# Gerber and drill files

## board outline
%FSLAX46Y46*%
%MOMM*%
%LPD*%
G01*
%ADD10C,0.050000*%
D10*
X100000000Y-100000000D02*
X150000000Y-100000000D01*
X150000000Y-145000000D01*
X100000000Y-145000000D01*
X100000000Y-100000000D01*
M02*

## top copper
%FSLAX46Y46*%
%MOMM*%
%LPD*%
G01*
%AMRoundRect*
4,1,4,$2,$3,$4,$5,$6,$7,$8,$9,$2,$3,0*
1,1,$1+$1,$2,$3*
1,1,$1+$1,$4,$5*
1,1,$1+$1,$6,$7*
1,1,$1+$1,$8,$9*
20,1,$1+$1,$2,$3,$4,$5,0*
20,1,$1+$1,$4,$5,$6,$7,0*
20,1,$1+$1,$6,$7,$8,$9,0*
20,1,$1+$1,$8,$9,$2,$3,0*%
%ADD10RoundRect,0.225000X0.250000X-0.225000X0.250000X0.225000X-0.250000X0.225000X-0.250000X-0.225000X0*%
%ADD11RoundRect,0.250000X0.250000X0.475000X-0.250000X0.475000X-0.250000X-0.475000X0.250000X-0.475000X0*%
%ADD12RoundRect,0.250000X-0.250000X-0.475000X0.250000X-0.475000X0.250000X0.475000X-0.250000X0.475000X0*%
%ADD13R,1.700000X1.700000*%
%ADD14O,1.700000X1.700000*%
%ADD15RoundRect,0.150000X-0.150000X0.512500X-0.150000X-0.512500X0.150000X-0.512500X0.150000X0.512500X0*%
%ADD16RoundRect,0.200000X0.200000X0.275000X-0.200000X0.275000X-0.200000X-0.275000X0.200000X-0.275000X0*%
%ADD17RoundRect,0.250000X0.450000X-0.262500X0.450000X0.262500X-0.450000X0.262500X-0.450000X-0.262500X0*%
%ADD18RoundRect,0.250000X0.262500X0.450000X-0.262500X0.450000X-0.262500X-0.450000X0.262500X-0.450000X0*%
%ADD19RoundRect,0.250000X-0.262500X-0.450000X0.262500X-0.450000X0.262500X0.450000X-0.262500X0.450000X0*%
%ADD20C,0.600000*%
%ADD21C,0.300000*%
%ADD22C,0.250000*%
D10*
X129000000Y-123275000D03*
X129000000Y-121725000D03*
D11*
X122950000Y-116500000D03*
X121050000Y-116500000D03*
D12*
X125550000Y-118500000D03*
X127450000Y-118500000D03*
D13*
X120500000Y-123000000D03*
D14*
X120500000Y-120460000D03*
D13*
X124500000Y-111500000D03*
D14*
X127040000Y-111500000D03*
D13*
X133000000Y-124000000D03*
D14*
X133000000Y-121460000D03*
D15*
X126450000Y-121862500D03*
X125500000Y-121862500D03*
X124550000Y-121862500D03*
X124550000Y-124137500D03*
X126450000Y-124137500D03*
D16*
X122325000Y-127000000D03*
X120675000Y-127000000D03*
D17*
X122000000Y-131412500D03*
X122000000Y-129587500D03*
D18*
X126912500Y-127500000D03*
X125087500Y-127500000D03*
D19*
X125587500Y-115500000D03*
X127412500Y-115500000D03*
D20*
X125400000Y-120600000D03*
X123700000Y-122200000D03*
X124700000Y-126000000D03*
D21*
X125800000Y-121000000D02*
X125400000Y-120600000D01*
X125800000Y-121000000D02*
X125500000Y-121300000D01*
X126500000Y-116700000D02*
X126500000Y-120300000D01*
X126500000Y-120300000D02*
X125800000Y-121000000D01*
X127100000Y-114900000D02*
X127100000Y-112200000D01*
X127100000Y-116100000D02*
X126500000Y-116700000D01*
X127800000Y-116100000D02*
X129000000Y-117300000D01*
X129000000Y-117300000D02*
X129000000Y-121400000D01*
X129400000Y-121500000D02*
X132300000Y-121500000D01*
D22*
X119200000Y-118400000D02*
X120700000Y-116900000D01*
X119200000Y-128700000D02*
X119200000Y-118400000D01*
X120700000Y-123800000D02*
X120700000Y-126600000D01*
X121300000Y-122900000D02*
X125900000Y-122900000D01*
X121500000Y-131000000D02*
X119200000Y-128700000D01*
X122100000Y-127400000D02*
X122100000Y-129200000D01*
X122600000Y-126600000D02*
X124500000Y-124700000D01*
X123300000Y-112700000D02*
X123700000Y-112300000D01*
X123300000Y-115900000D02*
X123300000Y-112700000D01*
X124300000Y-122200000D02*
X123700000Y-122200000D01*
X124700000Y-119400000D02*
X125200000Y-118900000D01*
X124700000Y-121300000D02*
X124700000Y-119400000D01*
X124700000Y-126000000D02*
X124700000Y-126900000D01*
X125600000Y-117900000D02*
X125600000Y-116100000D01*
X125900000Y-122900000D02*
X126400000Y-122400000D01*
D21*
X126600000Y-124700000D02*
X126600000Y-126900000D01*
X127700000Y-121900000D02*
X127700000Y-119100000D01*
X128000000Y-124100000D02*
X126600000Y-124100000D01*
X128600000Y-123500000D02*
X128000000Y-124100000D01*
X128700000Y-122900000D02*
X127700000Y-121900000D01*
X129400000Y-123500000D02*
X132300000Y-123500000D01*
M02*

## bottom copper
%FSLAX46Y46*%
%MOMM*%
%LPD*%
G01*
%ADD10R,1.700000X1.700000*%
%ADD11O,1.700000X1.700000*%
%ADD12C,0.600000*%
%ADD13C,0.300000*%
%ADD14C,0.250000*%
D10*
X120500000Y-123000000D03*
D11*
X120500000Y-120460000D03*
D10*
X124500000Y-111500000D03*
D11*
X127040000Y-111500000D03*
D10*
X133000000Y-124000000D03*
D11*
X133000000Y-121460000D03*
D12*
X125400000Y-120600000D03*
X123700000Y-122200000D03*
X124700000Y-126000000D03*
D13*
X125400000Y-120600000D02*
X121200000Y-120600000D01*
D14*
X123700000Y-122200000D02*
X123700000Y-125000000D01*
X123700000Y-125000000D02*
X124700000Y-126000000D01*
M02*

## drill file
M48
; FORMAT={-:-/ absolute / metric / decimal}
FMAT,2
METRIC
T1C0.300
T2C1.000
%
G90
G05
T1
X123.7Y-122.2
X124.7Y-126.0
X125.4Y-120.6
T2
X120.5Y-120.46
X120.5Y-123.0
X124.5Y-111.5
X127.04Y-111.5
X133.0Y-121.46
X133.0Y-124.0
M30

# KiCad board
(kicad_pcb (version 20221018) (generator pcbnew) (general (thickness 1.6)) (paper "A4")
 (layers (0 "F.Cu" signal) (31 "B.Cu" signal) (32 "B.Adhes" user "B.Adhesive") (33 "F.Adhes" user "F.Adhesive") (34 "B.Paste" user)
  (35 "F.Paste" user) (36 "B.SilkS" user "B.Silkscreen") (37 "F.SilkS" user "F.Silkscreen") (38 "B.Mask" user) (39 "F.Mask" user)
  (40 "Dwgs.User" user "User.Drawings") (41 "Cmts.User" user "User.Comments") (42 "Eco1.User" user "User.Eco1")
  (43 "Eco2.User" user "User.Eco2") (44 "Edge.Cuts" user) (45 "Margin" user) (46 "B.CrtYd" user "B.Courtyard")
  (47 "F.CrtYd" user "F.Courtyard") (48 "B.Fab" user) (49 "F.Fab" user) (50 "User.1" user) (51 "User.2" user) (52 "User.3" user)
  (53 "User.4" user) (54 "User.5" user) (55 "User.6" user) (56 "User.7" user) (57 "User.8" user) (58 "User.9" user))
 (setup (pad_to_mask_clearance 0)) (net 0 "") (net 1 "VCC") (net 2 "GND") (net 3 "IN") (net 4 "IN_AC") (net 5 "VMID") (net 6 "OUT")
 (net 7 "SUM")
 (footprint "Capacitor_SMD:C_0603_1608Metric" (layer "F.Cu") (at 129 122.5 90)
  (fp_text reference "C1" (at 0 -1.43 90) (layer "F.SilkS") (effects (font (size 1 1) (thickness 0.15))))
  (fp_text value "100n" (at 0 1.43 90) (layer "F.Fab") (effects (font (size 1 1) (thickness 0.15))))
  (pad "1" smd roundrect (at -0.775 0 90) (size 0.9 0.95) (layers "F.Cu" "F.Paste" "F.Mask") (roundrect_rratio 0.25) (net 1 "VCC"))
  (pad "2" smd roundrect (at 0.775 0 90) (size 0.9 0.95) (layers "F.Cu" "F.Paste" "F.Mask") (roundrect_rratio 0.25) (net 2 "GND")))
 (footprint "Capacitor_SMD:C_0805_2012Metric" (layer "F.Cu") (at 122 116.5 180)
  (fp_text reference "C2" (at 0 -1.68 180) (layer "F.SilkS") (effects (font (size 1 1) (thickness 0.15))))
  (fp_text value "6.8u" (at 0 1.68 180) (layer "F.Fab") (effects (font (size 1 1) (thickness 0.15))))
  (pad "1" smd roundrect (at -0.95 0 180) (size 1 1.45) (layers "F.Cu" "F.Paste" "F.Mask") (roundrect_rratio 0.25) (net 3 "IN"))
  (pad "2" smd roundrect (at 0.95 0 180) (size 1 1.45) (layers "F.Cu" "F.Paste" "F.Mask") (roundrect_rratio 0.25) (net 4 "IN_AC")))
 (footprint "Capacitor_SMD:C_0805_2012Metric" (layer "F.Cu") (at 126.5 118.5)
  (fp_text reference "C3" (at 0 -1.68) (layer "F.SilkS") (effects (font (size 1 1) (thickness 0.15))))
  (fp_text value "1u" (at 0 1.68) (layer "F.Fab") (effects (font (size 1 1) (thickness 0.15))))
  (pad "1" smd roundrect (at -0.95 0) (size 1 1.45) (layers "F.Cu" "F.Paste" "F.Mask") (roundrect_rratio 0.25) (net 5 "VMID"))
  (pad "2" smd roundrect (at 0.95 0) (size 1 1.45) (layers "F.Cu" "F.Paste" "F.Mask") (roundrect_rratio 0.25) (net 1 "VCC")))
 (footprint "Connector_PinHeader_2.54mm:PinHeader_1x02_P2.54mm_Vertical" (layer "F.Cu") (at 120.5 123 180)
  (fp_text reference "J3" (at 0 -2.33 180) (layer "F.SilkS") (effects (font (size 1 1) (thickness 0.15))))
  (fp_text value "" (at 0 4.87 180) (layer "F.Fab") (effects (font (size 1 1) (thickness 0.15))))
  (pad "1" thru_hole rect (at 0 0 180) (size 1.7 1.7) (drill 1) (layers "*.Cu" "*.Mask") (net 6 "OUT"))
  (pad "2" thru_hole oval (at 0 2.54 180) (size 1.7 1.7) (drill 1) (layers "*.Cu" "*.Mask") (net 2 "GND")))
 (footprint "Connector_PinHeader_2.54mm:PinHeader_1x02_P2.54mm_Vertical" (layer "F.Cu") (at 124.5 111.5 90)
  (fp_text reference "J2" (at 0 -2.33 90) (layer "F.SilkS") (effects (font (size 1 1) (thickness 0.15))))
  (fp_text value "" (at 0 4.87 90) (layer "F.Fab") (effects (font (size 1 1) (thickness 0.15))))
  (pad "1" thru_hole rect (at 0 0 90) (size 1.7 1.7) (drill 1) (layers "*.Cu" "*.Mask") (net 3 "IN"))
  (pad "2" thru_hole oval (at 0 2.54 90) (size 1.7 1.7) (drill 1) (layers "*.Cu" "*.Mask") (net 2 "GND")))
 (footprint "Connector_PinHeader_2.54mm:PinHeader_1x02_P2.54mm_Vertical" (layer "F.Cu") (at 133 124 180)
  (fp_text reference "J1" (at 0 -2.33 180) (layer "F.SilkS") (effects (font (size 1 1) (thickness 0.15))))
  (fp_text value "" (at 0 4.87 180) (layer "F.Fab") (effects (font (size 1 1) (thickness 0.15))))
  (pad "1" thru_hole rect (at 0 0 180) (size 1.7 1.7) (drill 1) (layers "*.Cu" "*.Mask") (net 1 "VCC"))
  (pad "2" thru_hole oval (at 0 2.54 180) (size 1.7 1.7) (drill 1) (layers "*.Cu" "*.Mask") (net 2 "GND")))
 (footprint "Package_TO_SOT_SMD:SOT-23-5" (layer "F.Cu") (at 125.5 123 -90)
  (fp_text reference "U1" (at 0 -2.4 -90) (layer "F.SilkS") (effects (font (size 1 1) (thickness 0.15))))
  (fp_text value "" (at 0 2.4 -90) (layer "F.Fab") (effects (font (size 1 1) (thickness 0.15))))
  (pad "1" smd roundrect (at -1.1375 -0.95 270) (size 1.325 0.6) (layers "F.Cu" "F.Paste" "F.Mask") (roundrect_rratio 0.25) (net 6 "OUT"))
  (pad "2" smd roundrect (at -1.1375 0 270) (size 1.325 0.6) (layers "F.Cu" "F.Paste" "F.Mask") (roundrect_rratio 0.25) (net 2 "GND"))
  (pad "3" smd roundrect (at -1.1375 0.95 270) (size 1.325 0.6) (layers "F.Cu" "F.Paste" "F.Mask") (roundrect_rratio 0.25) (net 5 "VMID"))
  (pad "4" smd roundrect (at 1.1375 0.95 270) (size 1.325 0.6) (layers "F.Cu" "F.Paste" "F.Mask") (roundrect_rratio 0.25) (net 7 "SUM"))
  (pad "5" smd roundrect (at 1.1375 -0.95 270) (size 1.325 0.6) (layers "F.Cu" "F.Paste" "F.Mask") (roundrect_rratio 0.25) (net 1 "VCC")))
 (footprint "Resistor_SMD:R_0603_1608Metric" (layer "F.Cu") (at 121.5 127 180)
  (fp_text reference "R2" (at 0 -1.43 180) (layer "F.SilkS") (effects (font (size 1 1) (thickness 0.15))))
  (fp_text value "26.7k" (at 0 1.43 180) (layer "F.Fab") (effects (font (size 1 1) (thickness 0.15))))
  (pad "1" smd roundrect (at -0.825 0 180) (size 0.8 0.95) (layers "F.Cu" "F.Paste" "F.Mask") (roundrect_rratio 0.25) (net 7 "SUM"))
  (pad "2" smd roundrect (at 0.825 0 180) (size 0.8 0.95) (layers "F.Cu" "F.Paste" "F.Mask") (roundrect_rratio 0.25) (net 6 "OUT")))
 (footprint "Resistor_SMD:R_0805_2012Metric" (layer "F.Cu") (at 122 130.5 90)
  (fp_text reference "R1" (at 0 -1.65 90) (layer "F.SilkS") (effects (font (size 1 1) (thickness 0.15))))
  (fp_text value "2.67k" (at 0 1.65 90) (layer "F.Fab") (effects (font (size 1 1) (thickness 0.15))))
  (pad "1" smd roundrect (at -0.9125 0 90) (size 1.025 1.4) (layers "F.Cu" "F.Paste" "F.Mask") (roundrect_rratio 0.243902) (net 4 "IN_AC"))
  (pad "2" smd roundrect (at 0.9125 0 90) (size 1.025 1.4) (layers "F.Cu" "F.Paste" "F.Mask") (roundrect_rratio 0.243902) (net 7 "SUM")))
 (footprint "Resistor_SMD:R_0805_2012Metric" (layer "F.Cu") (at 126 127.5 180)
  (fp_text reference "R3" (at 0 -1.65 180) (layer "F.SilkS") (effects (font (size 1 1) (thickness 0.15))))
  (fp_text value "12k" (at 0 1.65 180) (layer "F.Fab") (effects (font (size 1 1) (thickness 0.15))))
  (pad "1" smd roundrect (at -0.9125 0 180) (size 1.025 1.4) (layers "F.Cu" "F.Paste" "F.Mask") (roundrect_rratio 0.243902) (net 1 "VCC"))
  (pad "2" smd roundrect (at 0.9125 0 180) (size 1.025 1.4) (layers "F.Cu" "F.Paste" "F.Mask") (roundrect_rratio 0.243902) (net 5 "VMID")))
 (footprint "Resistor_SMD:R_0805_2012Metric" (layer "F.Cu") (at 126.5 115.5)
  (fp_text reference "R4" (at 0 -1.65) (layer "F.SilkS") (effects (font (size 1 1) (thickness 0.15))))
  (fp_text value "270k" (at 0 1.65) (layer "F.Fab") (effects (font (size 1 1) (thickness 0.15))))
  (pad "1" smd roundrect (at -0.9125 0) (size 1.025 1.4) (layers "F.Cu" "F.Paste" "F.Mask") (roundrect_rratio 0.243902) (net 5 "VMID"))
  (pad "2" smd roundrect (at 0.9125 0) (size 1.025 1.4) (layers "F.Cu" "F.Paste" "F.Mask") (roundrect_rratio 0.243902) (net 2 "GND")))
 (gr_rect (start 100 100) (end 150 145) (stroke (width 0.05) (type default)) (fill none) (layer "Edge.Cuts"))
 (segment (start 125.8 121) (end 125.4 120.6) (width 0.3) (layer "F.Cu") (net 2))
 (segment (start 125.8 121) (end 125.5 121.3) (width 0.3) (layer "F.Cu") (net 2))
 (segment (start 126.5 116.7) (end 126.5 120.3) (width 0.3) (layer "F.Cu") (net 2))
 (segment (start 126.5 120.3) (end 125.8 121) (width 0.3) (layer "F.Cu") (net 2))
 (segment (start 127.1 114.9) (end 127.1 112.2) (width 0.3) (layer "F.Cu") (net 2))
 (segment (start 127.1 116.1) (end 126.5 116.7) (width 0.3) (layer "F.Cu") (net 2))
 (segment (start 127.8 116.1) (end 129 117.3) (width 0.3) (layer "F.Cu") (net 2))
 (segment (start 129 117.3) (end 129 121.4) (width 0.3) (layer "F.Cu") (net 2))
 (segment (start 129.4 121.5) (end 132.3 121.5) (width 0.3) (layer "F.Cu") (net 2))
 (via (at 125.4 120.6) (size 0.6) (drill 0.3) (layers "F.Cu" "B.Cu") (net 2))
 (segment (start 119.2 118.4) (end 120.7 116.9) (width 0.25) (layer "F.Cu") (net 4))
 (segment (start 119.2 128.7) (end 119.2 118.4) (width 0.25) (layer "F.Cu") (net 4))
 (segment (start 120.7 123.8) (end 120.7 126.6) (width 0.25) (layer "F.Cu") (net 6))
 (segment (start 121.3 122.9) (end 125.9 122.9) (width 0.25) (layer "F.Cu") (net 6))
 (segment (start 121.5 131) (end 119.2 128.7) (width 0.25) (layer "F.Cu") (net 4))
 (segment (start 122.1 127.4) (end 122.1 129.2) (width 0.25) (layer "F.Cu") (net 7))
 (segment (start 122.6 126.6) (end 124.5 124.7) (width 0.25) (layer "F.Cu") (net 7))
 (segment (start 123.3 112.7) (end 123.7 112.3) (width 0.25) (layer "F.Cu") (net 3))
 (segment (start 123.3 115.9) (end 123.3 112.7) (width 0.25) (layer "F.Cu") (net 3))
 (segment (start 124.3 122.2) (end 123.7 122.2) (width 0.25) (layer "F.Cu") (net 5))
 (segment (start 124.7 119.4) (end 125.2 118.9) (width 0.25) (layer "F.Cu") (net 5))
 (segment (start 124.7 121.3) (end 124.7 119.4) (width 0.25) (layer "F.Cu") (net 5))
 (segment (start 124.7 126) (end 124.7 126.9) (width 0.25) (layer "F.Cu") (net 5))
 (segment (start 125.4 120.6) (end 121.2 120.6) (width 0.3) (layer "B.Cu") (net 2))
 (segment (start 125.6 117.9) (end 125.6 116.1) (width 0.25) (layer "F.Cu") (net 5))
 (segment (start 125.9 122.9) (end 126.4 122.4) (width 0.25) (layer "F.Cu") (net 6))
 (segment (start 126.6 124.7) (end 126.6 126.9) (width 0.3) (layer "F.Cu") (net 1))
 (segment (start 127.7 121.9) (end 127.7 119.1) (width 0.3) (layer "F.Cu") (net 1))
 (segment (start 128 124.1) (end 126.6 124.1) (width 0.3) (layer "F.Cu") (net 1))
 (segment (start 128.6 123.5) (end 128 124.1) (width 0.3) (layer "F.Cu") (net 1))
 (segment (start 128.7 122.9) (end 127.7 121.9) (width 0.3) (layer "F.Cu") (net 1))
 (segment (start 129.4 123.5) (end 132.3 123.5) (width 0.3) (layer "F.Cu") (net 1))
 (via (at 123.7 122.2) (size 0.6) (drill 0.3) (layers "F.Cu" "B.Cu") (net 5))
 (via (at 124.7 126) (size 0.6) (drill 0.3) (layers "F.Cu" "B.Cu") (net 5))
 (segment (start 123.7 122.2) (end 123.7 125) (width 0.25) (layer "B.Cu") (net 5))
 (segment (start 123.7 125) (end 124.7 126) (width 0.25) (layer "B.Cu") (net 5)))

